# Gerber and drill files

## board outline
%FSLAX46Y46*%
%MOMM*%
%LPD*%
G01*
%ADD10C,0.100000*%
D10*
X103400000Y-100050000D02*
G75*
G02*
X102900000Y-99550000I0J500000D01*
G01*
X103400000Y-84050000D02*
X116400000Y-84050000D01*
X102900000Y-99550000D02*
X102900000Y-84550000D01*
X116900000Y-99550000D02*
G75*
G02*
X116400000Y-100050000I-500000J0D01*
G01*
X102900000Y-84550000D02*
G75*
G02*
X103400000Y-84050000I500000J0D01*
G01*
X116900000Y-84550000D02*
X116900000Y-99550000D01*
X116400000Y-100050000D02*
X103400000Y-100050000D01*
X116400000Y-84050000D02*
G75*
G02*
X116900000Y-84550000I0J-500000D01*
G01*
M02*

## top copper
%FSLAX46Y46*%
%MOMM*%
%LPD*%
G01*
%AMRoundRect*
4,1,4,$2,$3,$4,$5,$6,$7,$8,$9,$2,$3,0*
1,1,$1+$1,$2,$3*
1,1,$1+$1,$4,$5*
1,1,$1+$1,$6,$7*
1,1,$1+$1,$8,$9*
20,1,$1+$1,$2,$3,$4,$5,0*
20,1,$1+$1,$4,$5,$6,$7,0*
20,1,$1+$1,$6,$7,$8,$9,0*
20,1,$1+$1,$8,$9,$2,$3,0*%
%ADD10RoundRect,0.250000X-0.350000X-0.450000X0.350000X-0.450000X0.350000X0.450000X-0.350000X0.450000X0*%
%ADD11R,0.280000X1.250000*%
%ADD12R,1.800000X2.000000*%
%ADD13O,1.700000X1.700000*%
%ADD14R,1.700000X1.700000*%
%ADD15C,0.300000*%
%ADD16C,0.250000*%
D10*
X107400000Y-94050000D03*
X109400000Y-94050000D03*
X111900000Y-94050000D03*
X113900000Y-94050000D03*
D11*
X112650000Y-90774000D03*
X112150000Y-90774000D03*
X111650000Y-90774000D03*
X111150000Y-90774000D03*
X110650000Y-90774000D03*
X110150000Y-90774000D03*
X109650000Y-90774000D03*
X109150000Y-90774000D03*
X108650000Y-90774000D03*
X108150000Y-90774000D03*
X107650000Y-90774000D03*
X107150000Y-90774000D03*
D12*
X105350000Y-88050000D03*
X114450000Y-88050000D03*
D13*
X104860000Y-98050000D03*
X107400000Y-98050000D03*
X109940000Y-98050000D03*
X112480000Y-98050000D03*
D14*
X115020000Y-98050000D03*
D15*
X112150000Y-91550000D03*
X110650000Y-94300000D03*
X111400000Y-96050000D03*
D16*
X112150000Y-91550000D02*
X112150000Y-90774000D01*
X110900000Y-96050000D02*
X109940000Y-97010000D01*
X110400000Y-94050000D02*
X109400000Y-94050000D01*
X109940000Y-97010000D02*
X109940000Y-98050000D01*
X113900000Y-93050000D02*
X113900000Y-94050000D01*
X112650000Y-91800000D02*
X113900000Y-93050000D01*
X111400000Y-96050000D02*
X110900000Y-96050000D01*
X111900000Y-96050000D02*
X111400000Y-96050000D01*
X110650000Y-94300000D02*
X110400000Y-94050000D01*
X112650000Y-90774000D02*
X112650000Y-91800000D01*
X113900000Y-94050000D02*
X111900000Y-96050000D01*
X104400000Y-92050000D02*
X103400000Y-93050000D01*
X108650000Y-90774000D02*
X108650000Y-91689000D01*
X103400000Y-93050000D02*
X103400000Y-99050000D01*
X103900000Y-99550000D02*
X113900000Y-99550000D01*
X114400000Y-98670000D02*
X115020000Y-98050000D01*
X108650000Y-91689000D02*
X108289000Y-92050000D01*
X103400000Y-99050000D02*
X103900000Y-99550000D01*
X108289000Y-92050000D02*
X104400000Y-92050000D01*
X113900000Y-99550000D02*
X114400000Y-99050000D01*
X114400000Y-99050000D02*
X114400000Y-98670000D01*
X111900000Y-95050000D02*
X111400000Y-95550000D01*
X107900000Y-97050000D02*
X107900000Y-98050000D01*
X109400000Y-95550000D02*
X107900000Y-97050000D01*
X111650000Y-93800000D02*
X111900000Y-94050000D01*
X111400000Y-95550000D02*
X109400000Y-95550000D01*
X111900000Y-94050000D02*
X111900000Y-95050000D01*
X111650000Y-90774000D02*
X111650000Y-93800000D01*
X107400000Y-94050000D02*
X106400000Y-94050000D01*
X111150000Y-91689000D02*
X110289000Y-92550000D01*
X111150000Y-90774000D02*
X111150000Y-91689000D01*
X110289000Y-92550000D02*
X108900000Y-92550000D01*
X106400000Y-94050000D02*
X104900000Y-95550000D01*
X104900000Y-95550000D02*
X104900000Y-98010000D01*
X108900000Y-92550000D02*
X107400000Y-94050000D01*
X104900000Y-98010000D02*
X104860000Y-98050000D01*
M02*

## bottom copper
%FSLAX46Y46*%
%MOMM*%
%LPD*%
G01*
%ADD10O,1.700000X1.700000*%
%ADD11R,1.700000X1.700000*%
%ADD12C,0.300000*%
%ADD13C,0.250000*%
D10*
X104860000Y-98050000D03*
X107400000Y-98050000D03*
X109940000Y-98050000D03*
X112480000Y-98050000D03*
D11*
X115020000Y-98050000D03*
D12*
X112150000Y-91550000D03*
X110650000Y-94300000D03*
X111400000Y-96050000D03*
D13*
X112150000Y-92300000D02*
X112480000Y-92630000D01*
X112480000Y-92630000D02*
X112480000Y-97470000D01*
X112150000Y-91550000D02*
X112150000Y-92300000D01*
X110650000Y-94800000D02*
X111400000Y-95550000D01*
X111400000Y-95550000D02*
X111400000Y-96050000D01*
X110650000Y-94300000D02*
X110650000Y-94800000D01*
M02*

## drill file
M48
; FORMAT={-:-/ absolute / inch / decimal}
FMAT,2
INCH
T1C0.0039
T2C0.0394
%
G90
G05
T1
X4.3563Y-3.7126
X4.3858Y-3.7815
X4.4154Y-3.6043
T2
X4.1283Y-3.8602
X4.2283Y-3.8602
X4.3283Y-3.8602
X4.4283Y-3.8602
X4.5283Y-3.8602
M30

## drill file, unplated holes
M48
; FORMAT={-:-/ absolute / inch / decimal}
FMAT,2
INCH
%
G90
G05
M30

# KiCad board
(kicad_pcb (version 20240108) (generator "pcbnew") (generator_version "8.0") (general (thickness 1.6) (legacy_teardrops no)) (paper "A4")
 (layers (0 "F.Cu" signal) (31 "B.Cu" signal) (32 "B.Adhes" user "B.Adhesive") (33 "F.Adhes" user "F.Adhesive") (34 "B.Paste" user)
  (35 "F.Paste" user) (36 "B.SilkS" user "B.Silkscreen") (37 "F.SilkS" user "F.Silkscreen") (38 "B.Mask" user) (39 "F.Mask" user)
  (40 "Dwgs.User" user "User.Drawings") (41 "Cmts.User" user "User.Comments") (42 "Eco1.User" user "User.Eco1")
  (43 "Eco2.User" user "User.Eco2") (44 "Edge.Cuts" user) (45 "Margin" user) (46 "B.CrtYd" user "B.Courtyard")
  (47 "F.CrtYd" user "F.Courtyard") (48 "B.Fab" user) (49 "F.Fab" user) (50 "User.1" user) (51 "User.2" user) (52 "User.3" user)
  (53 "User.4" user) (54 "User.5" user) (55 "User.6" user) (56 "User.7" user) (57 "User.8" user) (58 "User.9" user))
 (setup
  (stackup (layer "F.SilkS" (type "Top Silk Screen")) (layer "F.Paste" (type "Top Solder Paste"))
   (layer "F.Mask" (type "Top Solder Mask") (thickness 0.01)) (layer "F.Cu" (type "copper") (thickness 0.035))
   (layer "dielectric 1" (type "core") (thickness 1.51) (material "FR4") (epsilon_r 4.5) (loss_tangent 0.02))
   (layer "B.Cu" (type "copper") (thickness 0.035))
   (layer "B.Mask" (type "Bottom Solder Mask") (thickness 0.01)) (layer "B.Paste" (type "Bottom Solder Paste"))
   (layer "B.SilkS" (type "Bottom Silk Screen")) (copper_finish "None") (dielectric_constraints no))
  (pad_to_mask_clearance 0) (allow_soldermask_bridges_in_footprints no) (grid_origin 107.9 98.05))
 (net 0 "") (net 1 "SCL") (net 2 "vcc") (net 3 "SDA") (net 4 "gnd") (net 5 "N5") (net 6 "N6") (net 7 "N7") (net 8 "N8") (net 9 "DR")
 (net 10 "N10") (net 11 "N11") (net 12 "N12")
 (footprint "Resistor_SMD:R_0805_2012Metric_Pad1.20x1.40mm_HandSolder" (layer "F.Cu") (at 108.4 94.05)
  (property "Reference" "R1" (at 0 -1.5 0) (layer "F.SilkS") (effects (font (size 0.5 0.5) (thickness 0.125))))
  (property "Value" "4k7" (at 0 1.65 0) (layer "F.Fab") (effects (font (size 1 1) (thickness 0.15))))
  (pad "1" smd roundrect (at -1 0) (size 1.2 1.4) (layers "F.Cu" "F.Paste" "F.Mask") (roundrect_rratio 0.208333) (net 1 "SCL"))
  (pad "2" smd roundrect (at 1 0) (size 1.2 1.4) (layers "F.Cu" "F.Paste" "F.Mask") (roundrect_rratio 0.208333) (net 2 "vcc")))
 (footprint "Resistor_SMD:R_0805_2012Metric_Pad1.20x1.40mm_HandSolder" (layer "F.Cu") (at 112.9 94.05)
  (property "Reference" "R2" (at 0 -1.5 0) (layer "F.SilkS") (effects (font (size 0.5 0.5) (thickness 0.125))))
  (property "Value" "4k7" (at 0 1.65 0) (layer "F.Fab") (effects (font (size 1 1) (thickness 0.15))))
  (pad "1" smd roundrect (at -1 0) (size 1.2 1.4) (layers "F.Cu" "F.Paste" "F.Mask") (roundrect_rratio 0.208333) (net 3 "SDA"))
  (pad "2" smd roundrect (at 1 0) (size 1.2 1.4) (layers "F.Cu" "F.Paste" "F.Mask") (roundrect_rratio 0.208333) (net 2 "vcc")))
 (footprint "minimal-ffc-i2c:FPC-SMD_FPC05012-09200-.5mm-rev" (layer "F.Cu") (at 109.9 89.412 180)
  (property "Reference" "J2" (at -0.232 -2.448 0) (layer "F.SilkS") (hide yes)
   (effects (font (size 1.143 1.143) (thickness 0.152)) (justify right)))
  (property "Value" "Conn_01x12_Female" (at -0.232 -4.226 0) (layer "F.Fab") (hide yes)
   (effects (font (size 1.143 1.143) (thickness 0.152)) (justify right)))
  (pad "1" smd rect (at -2.75 -1.362 180) (size 0.28 1.25) (layers "F.Cu" "F.Paste" "F.Mask") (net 2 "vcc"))
  (pad "2" smd rect (at -2.25 -1.362 180) (size 0.28 1.25) (layers "F.Cu" "F.Paste" "F.Mask") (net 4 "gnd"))
  (pad "3" smd rect (at -1.75 -1.362 180) (size 0.28 1.25) (layers "F.Cu" "F.Paste" "F.Mask") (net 3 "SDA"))
  (pad "4" smd rect (at -1.25 -1.362 180) (size 0.28 1.25) (layers "F.Cu" "F.Paste" "F.Mask") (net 1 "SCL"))
  (pad "5" smd rect (at -0.75 -1.362 180) (size 0.28 1.25) (layers "F.Cu" "F.Paste" "F.Mask") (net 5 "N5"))
  (pad "6" smd rect (at -0.25 -1.362 180) (size 0.28 1.25) (layers "F.Cu" "F.Paste" "F.Mask") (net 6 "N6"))
  (pad "7" smd rect (at 0.25 -1.362 180) (size 0.28 1.25) (layers "F.Cu" "F.Paste" "F.Mask") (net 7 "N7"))
  (pad "8" smd rect (at 0.75 -1.362 180) (size 0.28 1.25) (layers "F.Cu" "F.Paste" "F.Mask") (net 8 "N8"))
  (pad "9" smd rect (at 1.25 -1.362 180) (size 0.28 1.25) (layers "F.Cu" "F.Paste" "F.Mask") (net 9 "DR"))
  (pad "10" smd rect (at 1.75 -1.362 180) (size 0.28 1.25) (layers "F.Cu" "F.Paste" "F.Mask") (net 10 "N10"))
  (pad "11" smd rect (at 2.25 -1.362 180) (size 0.28 1.25) (layers "F.Cu" "F.Paste" "F.Mask") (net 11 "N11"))
  (pad "12" smd rect (at 2.75 -1.362 180) (size 0.28 1.25) (layers "F.Cu" "F.Paste" "F.Mask") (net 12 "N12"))
  (pad "13" smd rect (at 4.55 1.362 180) (size 1.8 2) (layers "F.Cu" "F.Paste" "F.Mask"))
  (pad "14" smd rect (at -4.55 1.362 180) (size 1.8 2) (layers "F.Cu" "F.Paste" "F.Mask")))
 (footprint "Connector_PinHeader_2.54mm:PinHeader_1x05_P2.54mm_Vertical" (layer "B.Cu") (at 115.02 98.05 90)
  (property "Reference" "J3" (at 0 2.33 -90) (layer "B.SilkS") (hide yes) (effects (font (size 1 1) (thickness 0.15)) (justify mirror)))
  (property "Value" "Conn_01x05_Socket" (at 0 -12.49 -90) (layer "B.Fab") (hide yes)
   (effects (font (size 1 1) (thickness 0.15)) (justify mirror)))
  (pad "1" thru_hole rect (at 0 0 90) (size 1.7 1.7) (drill 1) (layers "*.Cu" "*.Mask") (remove_unused_layers no) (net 9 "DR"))
  (pad "2" thru_hole oval (at 0 -2.54 90) (size 1.7 1.7) (drill 1) (layers "*.Cu" "*.Mask") (remove_unused_layers no) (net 4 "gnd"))
  (pad "3" thru_hole oval (at 0 -5.08 90) (size 1.7 1.7) (drill 1) (layers "*.Cu" "*.Mask") (remove_unused_layers no) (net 2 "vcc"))
  (pad "4" thru_hole oval (at 0 -7.62 90) (size 1.7 1.7) (drill 1) (layers "*.Cu" "*.Mask") (remove_unused_layers no) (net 3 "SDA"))
  (pad "5" thru_hole oval (at 0 -10.16 90) (size 1.7 1.7) (drill 1) (layers "*.Cu" "*.Mask") (remove_unused_layers no) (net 1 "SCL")))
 (gr_arc (start 103.4 100.05) (mid 103.046447 99.903553) (end 102.9 99.55) (stroke (width 0.1) (type default)) (layer "Edge.Cuts"))
 (gr_line (start 103.4 84.05) (end 116.4 84.05) (stroke (width 0.1) (type default)) (layer "Edge.Cuts"))
 (gr_line (start 102.9 99.55) (end 102.9 84.55) (stroke (width 0.1) (type default)) (layer "Edge.Cuts"))
 (gr_arc (start 116.9 99.55) (mid 116.753553 99.903553) (end 116.4 100.05) (stroke (width 0.1) (type default)) (layer "Edge.Cuts"))
 (gr_arc (start 102.9 84.55) (mid 103.046447 84.196447) (end 103.4 84.05) (stroke (width 0.1) (type default)) (layer "Edge.Cuts"))
 (gr_line (start 116.9 84.55) (end 116.9 99.55) (stroke (width 0.1) (type default)) (layer "Edge.Cuts"))
 (gr_line (start 116.4 100.05) (end 103.4 100.05) (stroke (width 0.1) (type default)) (layer "Edge.Cuts"))
 (gr_arc (start 116.4 84.05) (mid 116.753553 84.196447) (end 116.9 84.55) (stroke (width 0.1) (type default)) (layer "Edge.Cuts"))
 (segment (start 112.15 91.55) (end 112.15 90.774) (width 0.25) (layer "F.Cu") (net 4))
 (via (at 112.15 91.55) (size 0.3) (drill 0.1) (layers "F.Cu" "B.Cu") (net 4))
 (segment (start 112.15 92.3) (end 112.48 92.63) (width 0.25) (layer "B.Cu") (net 4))
 (segment (start 112.48 92.63) (end 112.48 97.47) (width 0.25) (layer "B.Cu") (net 4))
 (segment (start 112.15 91.55) (end 112.15 92.3) (width 0.25) (layer "B.Cu") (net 4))
 (segment (start 110.9 96.05) (end 109.94 97.01) (width 0.25) (layer "F.Cu") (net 2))
 (segment (start 110.4 94.05) (end 109.4 94.05) (width 0.25) (layer "F.Cu") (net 2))
 (segment (start 109.94 97.01) (end 109.94 98.05) (width 0.25) (layer "F.Cu") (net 2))
 (segment (start 113.9 93.05) (end 113.9 94.05) (width 0.25) (layer "F.Cu") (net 2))
 (segment (start 112.65 91.8) (end 113.9 93.05) (width 0.25) (layer "F.Cu") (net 2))
 (segment (start 111.4 96.05) (end 110.9 96.05) (width 0.25) (layer "F.Cu") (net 2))
 (segment (start 111.9 96.05) (end 111.4 96.05) (width 0.25) (layer "F.Cu") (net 2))
 (segment (start 110.65 94.3) (end 110.4 94.05) (width 0.25) (layer "F.Cu") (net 2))
 (segment (start 112.65 90.774) (end 112.65 91.8) (width 0.25) (layer "F.Cu") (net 2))
 (segment (start 113.9 94.05) (end 111.9 96.05) (width 0.25) (layer "F.Cu") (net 2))
 (via (at 110.65 94.3) (size 0.3) (drill 0.1) (layers "F.Cu" "B.Cu") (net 2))
 (via (at 111.4 96.05) (size 0.3) (drill 0.1) (layers "F.Cu" "B.Cu") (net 2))
 (segment (start 110.65 94.8) (end 111.4 95.55) (width 0.25) (layer "B.Cu") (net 2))
 (segment (start 111.4 95.55) (end 111.4 96.05) (width 0.25) (layer "B.Cu") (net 2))
 (segment (start 110.65 94.3) (end 110.65 94.8) (width 0.25) (layer "B.Cu") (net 2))
 (segment (start 104.4 92.05) (end 103.4 93.05) (width 0.25) (layer "F.Cu") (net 9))
 (segment (start 108.65 90.774) (end 108.65 91.689) (width 0.25) (layer "F.Cu") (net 9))
 (segment (start 103.4 93.05) (end 103.4 99.05) (width 0.25) (layer "F.Cu") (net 9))
 (segment (start 103.9 99.55) (end 113.9 99.55) (width 0.25) (layer "F.Cu") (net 9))
 (segment (start 114.4 98.67) (end 115.02 98.05) (width 0.25) (layer "F.Cu") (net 9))
 (segment (start 108.65 91.689) (end 108.289 92.05) (width 0.25) (layer "F.Cu") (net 9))
 (segment (start 103.4 99.05) (end 103.9 99.55) (width 0.25) (layer "F.Cu") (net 9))
 (segment (start 108.289 92.05) (end 104.4 92.05) (width 0.25) (layer "F.Cu") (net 9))
 (segment (start 113.9 99.55) (end 114.4 99.05) (width 0.25) (layer "F.Cu") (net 9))
 (segment (start 114.4 99.05) (end 114.4 98.67) (width 0.25) (layer "F.Cu") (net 9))
 (segment (start 111.9 95.05) (end 111.4 95.55) (width 0.25) (layer "F.Cu") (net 3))
 (segment (start 107.9 97.05) (end 107.9 98.05) (width 0.25) (layer "F.Cu") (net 3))
 (segment (start 109.4 95.55) (end 107.9 97.05) (width 0.25) (layer "F.Cu") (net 3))
 (segment (start 111.65 93.8) (end 111.9 94.05) (width 0.25) (layer "F.Cu") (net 3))
 (segment (start 111.4 95.55) (end 109.4 95.55) (width 0.25) (layer "F.Cu") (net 3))
 (segment (start 111.9 94.05) (end 111.9 95.05) (width 0.25) (layer "F.Cu") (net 3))
 (segment (start 111.65 90.774) (end 111.65 93.8) (width 0.25) (layer "F.Cu") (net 3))
 (segment (start 107.4 94.05) (end 106.4 94.05) (width 0.25) (layer "F.Cu") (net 1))
 (segment (start 111.15 91.689) (end 110.289 92.55) (width 0.25) (layer "F.Cu") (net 1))
 (segment (start 111.15 90.774) (end 111.15 91.689) (width 0.25) (layer "F.Cu") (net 1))
 (segment (start 110.289 92.55) (end 108.9 92.55) (width 0.25) (layer "F.Cu") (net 1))
 (segment (start 106.4 94.05) (end 104.9 95.55) (width 0.25) (layer "F.Cu") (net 1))
 (segment (start 104.9 95.55) (end 104.9 98.01) (width 0.25) (layer "F.Cu") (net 1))
 (segment (start 108.9 92.55) (end 107.4 94.05) (width 0.25) (layer "F.Cu") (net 1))
 (segment (start 104.9 98.01) (end 104.86 98.05) (width 0.25) (layer "F.Cu") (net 1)))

